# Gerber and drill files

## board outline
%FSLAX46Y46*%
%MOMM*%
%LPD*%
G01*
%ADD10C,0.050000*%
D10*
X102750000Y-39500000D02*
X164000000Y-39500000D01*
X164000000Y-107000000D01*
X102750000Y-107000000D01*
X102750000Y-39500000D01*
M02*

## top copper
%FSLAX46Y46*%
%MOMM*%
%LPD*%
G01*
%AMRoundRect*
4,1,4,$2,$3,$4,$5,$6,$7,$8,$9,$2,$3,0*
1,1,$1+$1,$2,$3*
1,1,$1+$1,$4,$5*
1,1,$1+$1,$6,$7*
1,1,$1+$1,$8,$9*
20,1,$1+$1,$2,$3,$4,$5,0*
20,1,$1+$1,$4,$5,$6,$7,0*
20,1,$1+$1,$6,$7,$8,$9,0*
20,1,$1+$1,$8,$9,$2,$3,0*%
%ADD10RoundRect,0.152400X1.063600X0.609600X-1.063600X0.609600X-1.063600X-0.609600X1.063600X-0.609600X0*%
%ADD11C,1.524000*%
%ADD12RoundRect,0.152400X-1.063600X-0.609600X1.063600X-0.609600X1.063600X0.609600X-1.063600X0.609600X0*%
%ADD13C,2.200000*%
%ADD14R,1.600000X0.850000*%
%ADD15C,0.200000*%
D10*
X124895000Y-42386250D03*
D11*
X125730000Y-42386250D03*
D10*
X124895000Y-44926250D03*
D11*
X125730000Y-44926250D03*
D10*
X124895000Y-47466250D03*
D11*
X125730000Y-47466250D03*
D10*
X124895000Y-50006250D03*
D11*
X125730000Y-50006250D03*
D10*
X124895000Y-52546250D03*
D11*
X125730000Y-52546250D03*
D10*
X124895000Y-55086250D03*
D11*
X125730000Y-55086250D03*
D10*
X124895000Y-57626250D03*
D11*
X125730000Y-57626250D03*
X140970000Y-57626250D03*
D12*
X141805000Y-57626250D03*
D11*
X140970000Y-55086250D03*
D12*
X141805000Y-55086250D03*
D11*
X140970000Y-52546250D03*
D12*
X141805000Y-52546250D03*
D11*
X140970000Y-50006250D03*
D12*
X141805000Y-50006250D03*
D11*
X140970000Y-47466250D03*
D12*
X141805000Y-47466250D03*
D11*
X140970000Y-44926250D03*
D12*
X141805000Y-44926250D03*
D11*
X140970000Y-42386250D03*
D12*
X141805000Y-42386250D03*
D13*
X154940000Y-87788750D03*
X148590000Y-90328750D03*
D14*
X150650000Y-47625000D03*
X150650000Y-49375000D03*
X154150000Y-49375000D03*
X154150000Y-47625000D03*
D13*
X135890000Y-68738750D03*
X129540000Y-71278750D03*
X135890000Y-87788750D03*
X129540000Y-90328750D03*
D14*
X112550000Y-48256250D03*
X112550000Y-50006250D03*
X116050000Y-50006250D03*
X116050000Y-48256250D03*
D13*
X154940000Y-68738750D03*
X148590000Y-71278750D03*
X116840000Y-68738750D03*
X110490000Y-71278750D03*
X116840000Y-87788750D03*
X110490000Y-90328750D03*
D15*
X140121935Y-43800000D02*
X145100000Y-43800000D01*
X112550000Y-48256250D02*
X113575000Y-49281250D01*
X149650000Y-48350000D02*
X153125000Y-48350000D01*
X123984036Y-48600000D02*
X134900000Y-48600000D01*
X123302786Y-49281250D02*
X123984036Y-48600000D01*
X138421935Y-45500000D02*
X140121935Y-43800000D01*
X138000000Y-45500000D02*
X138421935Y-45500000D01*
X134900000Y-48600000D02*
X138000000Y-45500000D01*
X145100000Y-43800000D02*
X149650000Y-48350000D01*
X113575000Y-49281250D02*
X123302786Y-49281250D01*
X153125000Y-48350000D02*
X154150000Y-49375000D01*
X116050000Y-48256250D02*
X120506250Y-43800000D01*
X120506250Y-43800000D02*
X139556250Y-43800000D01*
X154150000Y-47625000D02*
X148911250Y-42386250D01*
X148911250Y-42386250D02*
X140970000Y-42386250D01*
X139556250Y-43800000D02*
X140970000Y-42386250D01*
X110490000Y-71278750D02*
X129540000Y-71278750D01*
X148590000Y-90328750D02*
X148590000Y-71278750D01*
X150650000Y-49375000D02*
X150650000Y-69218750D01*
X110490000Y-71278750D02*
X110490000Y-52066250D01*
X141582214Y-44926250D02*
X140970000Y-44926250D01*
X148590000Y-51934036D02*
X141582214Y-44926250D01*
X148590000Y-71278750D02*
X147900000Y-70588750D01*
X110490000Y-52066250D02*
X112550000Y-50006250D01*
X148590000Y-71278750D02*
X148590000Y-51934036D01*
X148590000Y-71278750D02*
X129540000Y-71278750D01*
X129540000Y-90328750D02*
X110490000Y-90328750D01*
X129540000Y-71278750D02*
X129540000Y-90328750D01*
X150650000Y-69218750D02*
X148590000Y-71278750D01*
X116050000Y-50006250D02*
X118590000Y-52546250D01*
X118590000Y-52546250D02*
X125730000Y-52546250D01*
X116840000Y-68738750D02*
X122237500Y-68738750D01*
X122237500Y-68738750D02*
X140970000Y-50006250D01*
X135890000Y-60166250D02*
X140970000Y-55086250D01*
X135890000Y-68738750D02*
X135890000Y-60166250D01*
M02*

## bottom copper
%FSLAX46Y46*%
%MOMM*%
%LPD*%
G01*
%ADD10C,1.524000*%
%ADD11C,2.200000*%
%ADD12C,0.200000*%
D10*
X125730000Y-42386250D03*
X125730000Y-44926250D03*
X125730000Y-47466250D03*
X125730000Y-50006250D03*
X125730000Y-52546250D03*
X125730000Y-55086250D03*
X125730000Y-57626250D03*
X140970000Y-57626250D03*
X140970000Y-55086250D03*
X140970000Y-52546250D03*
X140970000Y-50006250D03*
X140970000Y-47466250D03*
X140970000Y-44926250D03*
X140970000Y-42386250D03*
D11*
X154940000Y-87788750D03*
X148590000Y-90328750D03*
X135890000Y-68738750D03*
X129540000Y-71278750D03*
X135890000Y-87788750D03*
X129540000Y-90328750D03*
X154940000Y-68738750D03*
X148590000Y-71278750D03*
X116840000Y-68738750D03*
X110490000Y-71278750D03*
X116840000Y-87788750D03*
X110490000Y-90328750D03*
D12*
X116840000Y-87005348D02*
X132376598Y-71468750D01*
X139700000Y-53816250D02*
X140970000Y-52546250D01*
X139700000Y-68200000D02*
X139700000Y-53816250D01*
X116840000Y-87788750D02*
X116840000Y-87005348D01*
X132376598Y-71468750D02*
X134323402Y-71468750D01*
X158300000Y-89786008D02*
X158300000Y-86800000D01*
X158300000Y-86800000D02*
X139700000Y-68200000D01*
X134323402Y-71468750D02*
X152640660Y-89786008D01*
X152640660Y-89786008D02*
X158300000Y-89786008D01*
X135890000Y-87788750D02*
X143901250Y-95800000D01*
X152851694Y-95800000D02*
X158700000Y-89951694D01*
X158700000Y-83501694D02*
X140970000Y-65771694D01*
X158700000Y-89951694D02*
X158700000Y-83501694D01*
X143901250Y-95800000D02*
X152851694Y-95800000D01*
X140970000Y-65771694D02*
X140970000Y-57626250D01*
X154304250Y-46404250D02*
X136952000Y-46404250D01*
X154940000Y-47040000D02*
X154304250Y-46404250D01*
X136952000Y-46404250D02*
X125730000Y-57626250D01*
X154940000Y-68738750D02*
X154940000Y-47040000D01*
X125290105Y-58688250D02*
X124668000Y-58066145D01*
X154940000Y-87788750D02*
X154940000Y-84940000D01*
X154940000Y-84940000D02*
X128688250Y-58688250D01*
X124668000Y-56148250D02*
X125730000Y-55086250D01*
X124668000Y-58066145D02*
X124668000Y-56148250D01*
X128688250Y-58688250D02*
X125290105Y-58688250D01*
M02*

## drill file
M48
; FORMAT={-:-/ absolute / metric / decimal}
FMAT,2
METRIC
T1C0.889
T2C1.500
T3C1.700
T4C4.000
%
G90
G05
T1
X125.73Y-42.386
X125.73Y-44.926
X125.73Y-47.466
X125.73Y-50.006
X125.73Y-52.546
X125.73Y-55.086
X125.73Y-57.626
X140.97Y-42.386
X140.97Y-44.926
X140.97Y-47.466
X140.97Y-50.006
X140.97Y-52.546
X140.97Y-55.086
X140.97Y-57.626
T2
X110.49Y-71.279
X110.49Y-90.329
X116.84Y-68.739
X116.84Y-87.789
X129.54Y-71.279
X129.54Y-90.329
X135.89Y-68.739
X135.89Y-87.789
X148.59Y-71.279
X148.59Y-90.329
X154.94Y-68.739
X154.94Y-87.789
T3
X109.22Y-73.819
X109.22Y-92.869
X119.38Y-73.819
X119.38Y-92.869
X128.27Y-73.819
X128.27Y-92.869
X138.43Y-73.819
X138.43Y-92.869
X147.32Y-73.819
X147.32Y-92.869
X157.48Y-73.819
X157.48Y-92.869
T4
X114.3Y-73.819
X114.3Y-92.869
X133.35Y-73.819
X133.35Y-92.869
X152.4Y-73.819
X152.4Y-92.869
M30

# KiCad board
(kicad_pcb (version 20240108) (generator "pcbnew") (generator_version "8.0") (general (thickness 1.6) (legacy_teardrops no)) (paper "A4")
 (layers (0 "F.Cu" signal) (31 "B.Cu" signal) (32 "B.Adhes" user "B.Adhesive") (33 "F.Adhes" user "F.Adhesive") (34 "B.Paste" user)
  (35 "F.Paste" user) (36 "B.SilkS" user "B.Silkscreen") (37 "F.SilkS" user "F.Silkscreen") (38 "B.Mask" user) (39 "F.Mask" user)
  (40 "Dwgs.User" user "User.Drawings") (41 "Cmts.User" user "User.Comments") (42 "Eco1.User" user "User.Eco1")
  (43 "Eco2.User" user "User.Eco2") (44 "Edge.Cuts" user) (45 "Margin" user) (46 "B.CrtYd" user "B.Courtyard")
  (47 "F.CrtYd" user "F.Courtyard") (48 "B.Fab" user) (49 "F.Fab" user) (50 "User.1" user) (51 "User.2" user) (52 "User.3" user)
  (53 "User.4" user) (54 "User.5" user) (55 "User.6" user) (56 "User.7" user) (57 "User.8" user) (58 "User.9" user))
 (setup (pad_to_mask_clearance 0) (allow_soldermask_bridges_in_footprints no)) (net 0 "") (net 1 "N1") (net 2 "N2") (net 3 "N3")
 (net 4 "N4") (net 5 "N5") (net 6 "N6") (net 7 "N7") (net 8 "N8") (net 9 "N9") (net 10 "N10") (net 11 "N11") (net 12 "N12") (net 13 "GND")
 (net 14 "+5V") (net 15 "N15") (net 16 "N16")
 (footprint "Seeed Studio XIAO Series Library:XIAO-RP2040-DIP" (layer "F.Cu") (at 133.35 50.00625)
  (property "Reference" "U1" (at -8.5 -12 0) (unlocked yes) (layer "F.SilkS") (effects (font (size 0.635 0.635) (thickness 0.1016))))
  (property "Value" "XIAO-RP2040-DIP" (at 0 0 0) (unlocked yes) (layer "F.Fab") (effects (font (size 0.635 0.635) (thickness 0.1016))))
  (pad "1" smd roundrect (at -8.455 -7.62 180) (size 2.432 1.524) (layers "F.Cu" "F.Mask") (roundrect_rratio 0.1) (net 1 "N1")
   (thermal_bridge_angle 45))
  (pad "1" thru_hole circle (at -7.62 -7.62 180) (size 1.524 1.524) (drill 0.889) (layers "*.Cu" "*.Mask") (remove_unused_layers no)
   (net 1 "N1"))
  (pad "2" smd roundrect (at -8.455 -5.08 180) (size 2.432 1.524) (layers "F.Cu" "F.Mask") (roundrect_rratio 0.1) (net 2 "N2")
   (thermal_bridge_angle 45))
  (pad "2" thru_hole circle (at -7.62 -5.08 180) (size 1.524 1.524) (drill 0.889) (layers "*.Cu" "*.Mask") (remove_unused_layers no)
   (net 2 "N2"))
  (pad "3" smd roundrect (at -8.455 -2.54 180) (size 2.432 1.524) (layers "F.Cu" "F.Mask") (roundrect_rratio 0.1) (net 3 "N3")
   (thermal_bridge_angle 45))
  (pad "3" thru_hole circle (at -7.62 -2.54 180) (size 1.524 1.524) (drill 0.889) (layers "*.Cu" "*.Mask") (remove_unused_layers no)
   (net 3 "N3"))
  (pad "4" smd roundrect (at -8.455 0 180) (size 2.432 1.524) (layers "F.Cu" "F.Mask") (roundrect_rratio 0.1) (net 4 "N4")
   (thermal_bridge_angle 45))
  (pad "4" thru_hole circle (at -7.62 0 180) (size 1.524 1.524) (drill 0.889) (layers "*.Cu" "*.Mask") (remove_unused_layers no)
   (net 4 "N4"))
  (pad "5" smd roundrect (at -8.455 2.54 180) (size 2.432 1.524) (layers "F.Cu" "F.Mask") (roundrect_rratio 0.1) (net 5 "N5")
   (thermal_bridge_angle 45))
  (pad "5" thru_hole circle (at -7.62 2.54 180) (size 1.524 1.524) (drill 0.889) (layers "*.Cu" "*.Mask") (remove_unused_layers no)
   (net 5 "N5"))
  (pad "6" smd roundrect (at -8.455 5.08 180) (size 2.432 1.524) (layers "F.Cu" "F.Mask") (roundrect_rratio 0.1) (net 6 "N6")
   (thermal_bridge_angle 45))
  (pad "6" thru_hole circle (at -7.62 5.08 180) (size 1.524 1.524) (drill 0.889) (layers "*.Cu" "*.Mask") (remove_unused_layers no)
   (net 6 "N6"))
  (pad "7" smd roundrect (at -8.455 7.62 180) (size 2.432 1.524) (layers "F.Cu" "F.Mask") (roundrect_rratio 0.1) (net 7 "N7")
   (thermal_bridge_angle 45))
  (pad "7" thru_hole circle (at -7.62 7.62 180) (size 1.524 1.524) (drill 0.889) (layers "*.Cu" "*.Mask") (remove_unused_layers no)
   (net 7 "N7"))
  (pad "8" thru_hole circle (at 7.62 7.62) (size 1.524 1.524) (drill 0.889) (layers "*.Cu" "*.Mask") (remove_unused_layers no) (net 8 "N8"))
  (pad "8" smd roundrect (at 8.455 7.62) (size 2.432 1.524) (layers "F.Cu" "F.Mask") (roundrect_rratio 0.1) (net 8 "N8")
   (thermal_bridge_angle 45))
  (pad "9" thru_hole circle (at 7.62 5.08) (size 1.524 1.524) (drill 0.889) (layers "*.Cu" "*.Mask") (remove_unused_layers no) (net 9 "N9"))
  (pad "9" smd roundrect (at 8.455 5.08) (size 2.432 1.524) (layers "F.Cu" "F.Mask") (roundrect_rratio 0.1) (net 9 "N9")
   (thermal_bridge_angle 45))
  (pad "10" thru_hole circle (at 7.62 2.54) (size 1.524 1.524) (drill 0.889) (layers "*.Cu" "*.Mask") (remove_unused_layers no)
   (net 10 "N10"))
  (pad "10" smd roundrect (at 8.455 2.54) (size 2.432 1.524) (layers "F.Cu" "F.Mask") (roundrect_rratio 0.1) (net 10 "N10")
   (thermal_bridge_angle 45))
  (pad "11" thru_hole circle (at 7.62 0) (size 1.524 1.524) (drill 0.889) (layers "*.Cu" "*.Mask") (remove_unused_layers no) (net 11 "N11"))
  (pad "11" smd roundrect (at 8.455 0) (size 2.432 1.524) (layers "F.Cu" "F.Mask") (roundrect_rratio 0.1) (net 11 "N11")
   (thermal_bridge_angle 45))
  (pad "12" thru_hole circle (at 7.62 -2.54) (size 1.524 1.524) (drill 0.889) (layers "*.Cu" "*.Mask") (remove_unused_layers no)
   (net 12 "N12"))
  (pad "12" smd roundrect (at 8.455 -2.54) (size 2.432 1.524) (layers "F.Cu" "F.Mask") (roundrect_rratio 0.1) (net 12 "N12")
   (thermal_bridge_angle 45))
  (pad "13" thru_hole circle (at 7.62 -5.08) (size 1.524 1.524) (drill 0.889) (layers "*.Cu" "*.Mask") (remove_unused_layers no)
   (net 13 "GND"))
  (pad "13" smd roundrect (at 8.455 -5.08) (size 2.432 1.524) (layers "F.Cu" "F.Mask") (roundrect_rratio 0.1) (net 13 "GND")
   (thermal_bridge_angle 45))
  (pad "14" thru_hole circle (at 7.62 -7.62) (size 1.524 1.524) (drill 0.889) (layers "*.Cu" "*.Mask") (remove_unused_layers no)
   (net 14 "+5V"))
  (pad "14" smd roundrect (at 8.455 -7.62) (size 2.432 1.524) (layers "F.Cu" "F.Mask") (roundrect_rratio 0.1) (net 14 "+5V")
   (thermal_bridge_angle 45)))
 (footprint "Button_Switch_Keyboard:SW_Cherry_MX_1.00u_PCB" (layer "F.Cu") (at 154.94 87.78875)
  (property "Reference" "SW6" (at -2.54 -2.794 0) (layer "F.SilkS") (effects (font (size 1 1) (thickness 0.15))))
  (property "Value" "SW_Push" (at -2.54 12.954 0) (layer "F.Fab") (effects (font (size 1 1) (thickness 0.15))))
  (pad "" np_thru_hole circle (at -7.62 5.08) (size 1.7 1.7) (drill 1.7) (layers "*.Cu" "*.Mask"))
  (pad "" np_thru_hole circle (at -2.54 5.08) (size 4 4) (drill 4) (layers "*.Cu" "*.Mask"))
  (pad "" np_thru_hole circle (at 2.54 5.08) (size 1.7 1.7) (drill 1.7) (layers "*.Cu" "*.Mask"))
  (pad "1" thru_hole circle (at 0 0) (size 2.2 2.2) (drill 1.5) (layers "*.Cu" "*.Mask") (remove_unused_layers no) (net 6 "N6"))
  (pad "2" thru_hole circle (at -6.35 2.54) (size 2.2 2.2) (drill 1.5) (layers "*.Cu" "*.Mask") (remove_unused_layers no) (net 13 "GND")))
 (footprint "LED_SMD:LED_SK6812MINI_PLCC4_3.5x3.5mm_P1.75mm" (layer "F.Cu") (at 152.4 48.5)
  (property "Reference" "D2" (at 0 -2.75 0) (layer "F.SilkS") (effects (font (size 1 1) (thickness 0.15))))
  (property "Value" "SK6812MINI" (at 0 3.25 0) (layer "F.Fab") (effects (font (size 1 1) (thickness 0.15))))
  (pad "1" smd rect (at -1.75 -0.875) (size 1.6 0.85) (layers "F.Cu" "F.Paste" "F.Mask") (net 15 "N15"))
  (pad "2" smd rect (at -1.75 0.875) (size 1.6 0.85) (layers "F.Cu" "F.Paste" "F.Mask") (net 13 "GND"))
  (pad "3" smd rect (at 1.75 0.875) (size 1.6 0.85) (layers "F.Cu" "F.Paste" "F.Mask") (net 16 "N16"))
  (pad "4" smd rect (at 1.75 -0.875) (size 1.6 0.85) (layers "F.Cu" "F.Paste" "F.Mask") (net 14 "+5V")))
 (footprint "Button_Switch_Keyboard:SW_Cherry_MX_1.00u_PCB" (layer "F.Cu") (at 135.89 68.73875)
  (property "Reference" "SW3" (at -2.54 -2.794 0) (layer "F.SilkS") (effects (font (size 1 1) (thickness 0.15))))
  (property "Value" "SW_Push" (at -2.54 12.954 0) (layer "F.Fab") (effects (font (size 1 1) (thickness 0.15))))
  (pad "" np_thru_hole circle (at -7.62 5.08) (size 1.7 1.7) (drill 1.7) (layers "*.Cu" "*.Mask"))
  (pad "" np_thru_hole circle (at -2.54 5.08) (size 4 4) (drill 4) (layers "*.Cu" "*.Mask"))
  (pad "" np_thru_hole circle (at 2.54 5.08) (size 1.7 1.7) (drill 1.7) (layers "*.Cu" "*.Mask"))
  (pad "1" thru_hole circle (at 0 0) (size 2.2 2.2) (drill 1.5) (layers "*.Cu" "*.Mask") (remove_unused_layers no) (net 9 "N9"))
  (pad "2" thru_hole circle (at -6.35 2.54) (size 2.2 2.2) (drill 1.5) (layers "*.Cu" "*.Mask") (remove_unused_layers no) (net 13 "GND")))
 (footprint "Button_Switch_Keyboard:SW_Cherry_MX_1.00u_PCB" (layer "F.Cu") (at 135.89 87.78875)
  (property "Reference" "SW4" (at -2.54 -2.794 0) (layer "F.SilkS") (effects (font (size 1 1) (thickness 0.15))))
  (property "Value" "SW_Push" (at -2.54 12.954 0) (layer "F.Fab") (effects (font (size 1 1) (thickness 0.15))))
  (pad "" np_thru_hole circle (at -7.62 5.08) (size 1.7 1.7) (drill 1.7) (layers "*.Cu" "*.Mask"))
  (pad "" np_thru_hole circle (at -2.54 5.08) (size 4 4) (drill 4) (layers "*.Cu" "*.Mask"))
  (pad "" np_thru_hole circle (at 2.54 5.08) (size 1.7 1.7) (drill 1.7) (layers "*.Cu" "*.Mask"))
  (pad "1" thru_hole circle (at 0 0) (size 2.2 2.2) (drill 1.5) (layers "*.Cu" "*.Mask") (remove_unused_layers no) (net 8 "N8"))
  (pad "2" thru_hole circle (at -6.35 2.54) (size 2.2 2.2) (drill 1.5) (layers "*.Cu" "*.Mask") (remove_unused_layers no) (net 13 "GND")))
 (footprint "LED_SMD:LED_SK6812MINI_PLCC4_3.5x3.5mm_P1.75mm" (layer "F.Cu") (at 114.3 49.13125)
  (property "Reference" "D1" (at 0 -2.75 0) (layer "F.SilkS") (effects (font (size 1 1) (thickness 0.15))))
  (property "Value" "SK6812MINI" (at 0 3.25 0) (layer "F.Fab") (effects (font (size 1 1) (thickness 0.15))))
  (pad "1" smd rect (at -1.75 -0.875) (size 1.6 0.85) (layers "F.Cu" "F.Paste" "F.Mask") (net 16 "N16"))
  (pad "2" smd rect (at -1.75 0.875) (size 1.6 0.85) (layers "F.Cu" "F.Paste" "F.Mask") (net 13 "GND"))
  (pad "3" smd rect (at 1.75 0.875) (size 1.6 0.85) (layers "F.Cu" "F.Paste" "F.Mask") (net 5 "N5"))
  (pad "4" smd rect (at 1.75 -0.875) (size 1.6 0.85) (layers "F.Cu" "F.Paste" "F.Mask") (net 14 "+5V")))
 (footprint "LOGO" (layer "F.Cu") (at 133.35 80.80375)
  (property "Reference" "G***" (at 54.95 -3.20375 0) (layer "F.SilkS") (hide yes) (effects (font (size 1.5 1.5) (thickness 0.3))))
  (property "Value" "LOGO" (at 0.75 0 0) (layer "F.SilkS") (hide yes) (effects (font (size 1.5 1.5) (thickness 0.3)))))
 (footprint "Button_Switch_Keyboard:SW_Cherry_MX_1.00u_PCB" (layer "F.Cu") (at 154.94 68.73875)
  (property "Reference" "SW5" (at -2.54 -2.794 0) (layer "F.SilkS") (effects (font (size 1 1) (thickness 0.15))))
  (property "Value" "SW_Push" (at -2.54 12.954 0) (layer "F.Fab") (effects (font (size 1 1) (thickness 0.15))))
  (pad "" np_thru_hole circle (at -7.62 5.08) (size 1.7 1.7) (drill 1.7) (layers "*.Cu" "*.Mask"))
  (pad "" np_thru_hole circle (at -2.54 5.08) (size 4 4) (drill 4) (layers "*.Cu" "*.Mask"))
  (pad "" np_thru_hole circle (at 2.54 5.08) (size 1.7 1.7) (drill 1.7) (layers "*.Cu" "*.Mask"))
  (pad "1" thru_hole circle (at 0 0) (size 2.2 2.2) (drill 1.5) (layers "*.Cu" "*.Mask") (remove_unused_layers no) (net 7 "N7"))
  (pad "2" thru_hole circle (at -6.35 2.54) (size 2.2 2.2) (drill 1.5) (layers "*.Cu" "*.Mask") (remove_unused_layers no) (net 13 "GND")))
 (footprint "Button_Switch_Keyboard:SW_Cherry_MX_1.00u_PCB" (layer "F.Cu") (at 116.84 68.73875)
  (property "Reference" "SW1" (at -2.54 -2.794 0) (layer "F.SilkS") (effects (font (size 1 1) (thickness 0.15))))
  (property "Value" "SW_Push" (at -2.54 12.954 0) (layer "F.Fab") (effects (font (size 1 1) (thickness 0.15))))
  (pad "" np_thru_hole circle (at -7.62 5.08) (size 1.7 1.7) (drill 1.7) (layers "*.Cu" "*.Mask"))
  (pad "" np_thru_hole circle (at -2.54 5.08) (size 4 4) (drill 4) (layers "*.Cu" "*.Mask"))
  (pad "" np_thru_hole circle (at 2.54 5.08) (size 1.7 1.7) (drill 1.7) (layers "*.Cu" "*.Mask"))
  (pad "1" thru_hole circle (at 0 0) (size 2.2 2.2) (drill 1.5) (layers "*.Cu" "*.Mask") (remove_unused_layers no) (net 11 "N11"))
  (pad "2" thru_hole circle (at -6.35 2.54) (size 2.2 2.2) (drill 1.5) (layers "*.Cu" "*.Mask") (remove_unused_layers no) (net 13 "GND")))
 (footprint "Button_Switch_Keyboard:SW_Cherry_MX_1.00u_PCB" (layer "F.Cu") (at 116.84 87.78875)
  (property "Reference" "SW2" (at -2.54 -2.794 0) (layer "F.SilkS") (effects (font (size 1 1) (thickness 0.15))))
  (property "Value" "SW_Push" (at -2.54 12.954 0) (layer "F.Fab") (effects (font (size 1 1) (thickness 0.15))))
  (pad "" np_thru_hole circle (at -7.62 5.08) (size 1.7 1.7) (drill 1.7) (layers "*.Cu" "*.Mask"))
  (pad "" np_thru_hole circle (at -2.54 5.08) (size 4 4) (drill 4) (layers "*.Cu" "*.Mask"))
  (pad "" np_thru_hole circle (at 2.54 5.08) (size 1.7 1.7) (drill 1.7) (layers "*.Cu" "*.Mask"))
  (pad "1" thru_hole circle (at 0 0) (size 2.2 2.2) (drill 1.5) (layers "*.Cu" "*.Mask") (remove_unused_layers no) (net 10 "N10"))
  (pad "2" thru_hole circle (at -6.35 2.54) (size 2.2 2.2) (drill 1.5) (layers "*.Cu" "*.Mask") (remove_unused_layers no) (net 13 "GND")))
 (gr_rect (start 102.75 39.5) (end 164 107) (stroke (width 0.05) (type default)) (fill none) (layer "Edge.Cuts"))
 (segment (start 140.121935 43.8) (end 145.1 43.8) (width 0.2) (layer "F.Cu") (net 16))
 (segment (start 112.55 48.25625) (end 113.575 49.28125) (width 0.2) (layer "F.Cu") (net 16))
 (segment (start 149.65 48.35) (end 153.125 48.35) (width 0.2) (layer "F.Cu") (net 16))
 (segment (start 123.984036 48.6) (end 134.9 48.6) (width 0.2) (layer "F.Cu") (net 16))
 (segment (start 123.302786 49.28125) (end 123.984036 48.6) (width 0.2) (layer "F.Cu") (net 16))
 (segment (start 138.421935 45.5) (end 140.121935 43.8) (width 0.2) (layer "F.Cu") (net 16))
 (segment (start 138 45.5) (end 138.421935 45.5) (width 0.2) (layer "F.Cu") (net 16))
 (segment (start 134.9 48.6) (end 138 45.5) (width 0.2) (layer "F.Cu") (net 16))
 (segment (start 145.1 43.8) (end 149.65 48.35) (width 0.2) (layer "F.Cu") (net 16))
 (segment (start 113.575 49.28125) (end 123.302786 49.28125) (width 0.2) (layer "F.Cu") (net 16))
 (segment (start 153.125 48.35) (end 154.15 49.375) (width 0.2) (layer "F.Cu") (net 16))
 (segment (start 116.05 48.25625) (end 120.50625 43.8) (width 0.2) (layer "F.Cu") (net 14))
 (segment (start 120.50625 43.8) (end 139.55625 43.8) (width 0.2) (layer "F.Cu") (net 14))
 (segment (start 154.15 47.625) (end 148.91125 42.38625) (width 0.2) (layer "F.Cu") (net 14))
 (segment (start 148.91125 42.38625) (end 140.97 42.38625) (width 0.2) (layer "F.Cu") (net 14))
 (segment (start 139.55625 43.8) (end 140.97 42.38625) (width 0.2) (layer "F.Cu") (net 14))
 (segment (start 110.49 71.27875) (end 129.54 71.27875) (width 0.2) (layer "F.Cu") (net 13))
 (segment (start 148.59 90.32875) (end 148.59 71.27875) (width 0.2) (layer "F.Cu") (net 13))
 (segment (start 150.65 49.375) (end 150.65 69.21875) (width 0.2) (layer "F.Cu") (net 13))
 (segment (start 110.49 71.27875) (end 110.49 52.06625) (width 0.2) (layer "F.Cu") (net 13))
 (segment (start 141.582214 44.92625) (end 140.97 44.92625) (width 0.2) (layer "F.Cu") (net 13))
 (segment (start 148.59 51.934036) (end 141.582214 44.92625) (width 0.2) (layer "F.Cu") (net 13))
 (segment (start 148.59 71.27875) (end 147.9 70.58875) (width 0.2) (layer "F.Cu") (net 13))
 (segment (start 110.49 52.06625) (end 112.55 50.00625) (width 0.2) (layer "F.Cu") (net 13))
 (segment (start 148.59 71.27875) (end 148.59 51.934036) (width 0.2) (layer "F.Cu") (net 13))
 (segment (start 148.59 71.27875) (end 129.54 71.27875) (width 0.2) (layer "F.Cu") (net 13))
 (segment (start 129.54 90.32875) (end 110.49 90.32875) (width 0.2) (layer "F.Cu") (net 13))
 (segment (start 129.54 71.27875) (end 129.54 90.32875) (width 0.2) (layer "F.Cu") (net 13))
 (segment (start 150.65 69.21875) (end 148.59 71.27875) (width 0.2) (layer "F.Cu") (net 13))
 (segment (start 116.05 50.00625) (end 118.59 52.54625) (width 0.2) (layer "F.Cu") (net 5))
 (segment (start 118.59 52.54625) (end 125.73 52.54625) (width 0.2) (layer "F.Cu") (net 5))
 (segment (start 116.84 68.73875) (end 122.2375 68.73875) (width 0.2) (layer "F.Cu") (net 11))
 (segment (start 122.2375 68.73875) (end 140.97 50.00625) (width 0.2) (layer "F.Cu") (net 11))
 (segment (start 116.84 87.005348) (end 132.376598 71.46875) (width 0.2) (layer "B.Cu") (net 10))
 (segment (start 139.7 53.81625) (end 140.97 52.54625) (width 0.2) (layer "B.Cu") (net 10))
 (segment (start 139.7 68.2) (end 139.7 53.81625) (width 0.2) (layer "B.Cu") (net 10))
 (segment (start 116.84 87.78875) (end 116.84 87.005348) (width 0.2) (layer "B.Cu") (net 10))
 (segment (start 132.376598 71.46875) (end 134.323402 71.46875) (width 0.2) (layer "B.Cu") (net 10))
 (segment (start 158.3 89.786008) (end 158.3 86.8) (width 0.2) (layer "B.Cu") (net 10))
 (segment (start 158.3 86.8) (end 139.7 68.2) (width 0.2) (layer "B.Cu") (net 10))
 (segment (start 134.323402 71.46875) (end 152.64066 89.786008) (width 0.2) (layer "B.Cu") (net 10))
 (segment (start 152.64066 89.786008) (end 158.3 89.786008) (width 0.2) (layer "B.Cu") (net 10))
 (segment (start 135.89 60.16625) (end 140.97 55.08625) (width 0.2) (layer "F.Cu") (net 9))
 (segment (start 135.89 68.73875) (end 135.89 60.16625) (width 0.2) (layer "F.Cu") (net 9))
 (segment (start 135.89 87.78875) (end 143.90125 95.8) (width 0.2) (layer "B.Cu") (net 8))
 (segment (start 152.851694 95.8) (end 158.7 89.951694) (width 0.2) (layer "B.Cu") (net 8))
 (segment (start 158.7 83.501694) (end 140.97 65.771694) (width 0.2) (layer "B.Cu") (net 8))
 (segment (start 158.7 89.951694) (end 158.7 83.501694) (width 0.2) (layer "B.Cu") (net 8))
 (segment (start 143.90125 95.8) (end 152.851694 95.8) (width 0.2) (layer "B.Cu") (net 8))
 (segment (start 140.97 65.771694) (end 140.97 57.62625) (width 0.2) (layer "B.Cu") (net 8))
 (segment (start 154.30425 46.40425) (end 136.952 46.40425) (width 0.2) (layer "B.Cu") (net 7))
 (segment (start 154.94 47.04) (end 154.30425 46.40425) (width 0.2) (layer "B.Cu") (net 7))
 (segment (start 136.952 46.40425) (end 125.73 57.62625) (width 0.2) (layer "B.Cu") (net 7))
 (segment (start 154.94 68.73875) (end 154.94 47.04) (width 0.2) (layer "B.Cu") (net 7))
 (segment (start 125.290105 58.68825) (end 124.668 58.066145) (width 0.2) (layer "B.Cu") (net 6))
 (segment (start 154.94 87.78875) (end 154.94 84.94) (width 0.2) (layer "B.Cu") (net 6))
 (segment (start 154.94 84.94) (end 128.68825 58.68825) (width 0.2) (layer "B.Cu") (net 6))
 (segment (start 124.668 56.14825) (end 125.73 55.08625) (width 0.2) (layer "B.Cu") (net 6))
 (segment (start 124.668 58.066145) (end 124.668 56.14825) (width 0.2) (layer "B.Cu") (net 6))
 (segment (start 128.68825 58.68825) (end 125.290105 58.68825) (width 0.2) (layer "B.Cu") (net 6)))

